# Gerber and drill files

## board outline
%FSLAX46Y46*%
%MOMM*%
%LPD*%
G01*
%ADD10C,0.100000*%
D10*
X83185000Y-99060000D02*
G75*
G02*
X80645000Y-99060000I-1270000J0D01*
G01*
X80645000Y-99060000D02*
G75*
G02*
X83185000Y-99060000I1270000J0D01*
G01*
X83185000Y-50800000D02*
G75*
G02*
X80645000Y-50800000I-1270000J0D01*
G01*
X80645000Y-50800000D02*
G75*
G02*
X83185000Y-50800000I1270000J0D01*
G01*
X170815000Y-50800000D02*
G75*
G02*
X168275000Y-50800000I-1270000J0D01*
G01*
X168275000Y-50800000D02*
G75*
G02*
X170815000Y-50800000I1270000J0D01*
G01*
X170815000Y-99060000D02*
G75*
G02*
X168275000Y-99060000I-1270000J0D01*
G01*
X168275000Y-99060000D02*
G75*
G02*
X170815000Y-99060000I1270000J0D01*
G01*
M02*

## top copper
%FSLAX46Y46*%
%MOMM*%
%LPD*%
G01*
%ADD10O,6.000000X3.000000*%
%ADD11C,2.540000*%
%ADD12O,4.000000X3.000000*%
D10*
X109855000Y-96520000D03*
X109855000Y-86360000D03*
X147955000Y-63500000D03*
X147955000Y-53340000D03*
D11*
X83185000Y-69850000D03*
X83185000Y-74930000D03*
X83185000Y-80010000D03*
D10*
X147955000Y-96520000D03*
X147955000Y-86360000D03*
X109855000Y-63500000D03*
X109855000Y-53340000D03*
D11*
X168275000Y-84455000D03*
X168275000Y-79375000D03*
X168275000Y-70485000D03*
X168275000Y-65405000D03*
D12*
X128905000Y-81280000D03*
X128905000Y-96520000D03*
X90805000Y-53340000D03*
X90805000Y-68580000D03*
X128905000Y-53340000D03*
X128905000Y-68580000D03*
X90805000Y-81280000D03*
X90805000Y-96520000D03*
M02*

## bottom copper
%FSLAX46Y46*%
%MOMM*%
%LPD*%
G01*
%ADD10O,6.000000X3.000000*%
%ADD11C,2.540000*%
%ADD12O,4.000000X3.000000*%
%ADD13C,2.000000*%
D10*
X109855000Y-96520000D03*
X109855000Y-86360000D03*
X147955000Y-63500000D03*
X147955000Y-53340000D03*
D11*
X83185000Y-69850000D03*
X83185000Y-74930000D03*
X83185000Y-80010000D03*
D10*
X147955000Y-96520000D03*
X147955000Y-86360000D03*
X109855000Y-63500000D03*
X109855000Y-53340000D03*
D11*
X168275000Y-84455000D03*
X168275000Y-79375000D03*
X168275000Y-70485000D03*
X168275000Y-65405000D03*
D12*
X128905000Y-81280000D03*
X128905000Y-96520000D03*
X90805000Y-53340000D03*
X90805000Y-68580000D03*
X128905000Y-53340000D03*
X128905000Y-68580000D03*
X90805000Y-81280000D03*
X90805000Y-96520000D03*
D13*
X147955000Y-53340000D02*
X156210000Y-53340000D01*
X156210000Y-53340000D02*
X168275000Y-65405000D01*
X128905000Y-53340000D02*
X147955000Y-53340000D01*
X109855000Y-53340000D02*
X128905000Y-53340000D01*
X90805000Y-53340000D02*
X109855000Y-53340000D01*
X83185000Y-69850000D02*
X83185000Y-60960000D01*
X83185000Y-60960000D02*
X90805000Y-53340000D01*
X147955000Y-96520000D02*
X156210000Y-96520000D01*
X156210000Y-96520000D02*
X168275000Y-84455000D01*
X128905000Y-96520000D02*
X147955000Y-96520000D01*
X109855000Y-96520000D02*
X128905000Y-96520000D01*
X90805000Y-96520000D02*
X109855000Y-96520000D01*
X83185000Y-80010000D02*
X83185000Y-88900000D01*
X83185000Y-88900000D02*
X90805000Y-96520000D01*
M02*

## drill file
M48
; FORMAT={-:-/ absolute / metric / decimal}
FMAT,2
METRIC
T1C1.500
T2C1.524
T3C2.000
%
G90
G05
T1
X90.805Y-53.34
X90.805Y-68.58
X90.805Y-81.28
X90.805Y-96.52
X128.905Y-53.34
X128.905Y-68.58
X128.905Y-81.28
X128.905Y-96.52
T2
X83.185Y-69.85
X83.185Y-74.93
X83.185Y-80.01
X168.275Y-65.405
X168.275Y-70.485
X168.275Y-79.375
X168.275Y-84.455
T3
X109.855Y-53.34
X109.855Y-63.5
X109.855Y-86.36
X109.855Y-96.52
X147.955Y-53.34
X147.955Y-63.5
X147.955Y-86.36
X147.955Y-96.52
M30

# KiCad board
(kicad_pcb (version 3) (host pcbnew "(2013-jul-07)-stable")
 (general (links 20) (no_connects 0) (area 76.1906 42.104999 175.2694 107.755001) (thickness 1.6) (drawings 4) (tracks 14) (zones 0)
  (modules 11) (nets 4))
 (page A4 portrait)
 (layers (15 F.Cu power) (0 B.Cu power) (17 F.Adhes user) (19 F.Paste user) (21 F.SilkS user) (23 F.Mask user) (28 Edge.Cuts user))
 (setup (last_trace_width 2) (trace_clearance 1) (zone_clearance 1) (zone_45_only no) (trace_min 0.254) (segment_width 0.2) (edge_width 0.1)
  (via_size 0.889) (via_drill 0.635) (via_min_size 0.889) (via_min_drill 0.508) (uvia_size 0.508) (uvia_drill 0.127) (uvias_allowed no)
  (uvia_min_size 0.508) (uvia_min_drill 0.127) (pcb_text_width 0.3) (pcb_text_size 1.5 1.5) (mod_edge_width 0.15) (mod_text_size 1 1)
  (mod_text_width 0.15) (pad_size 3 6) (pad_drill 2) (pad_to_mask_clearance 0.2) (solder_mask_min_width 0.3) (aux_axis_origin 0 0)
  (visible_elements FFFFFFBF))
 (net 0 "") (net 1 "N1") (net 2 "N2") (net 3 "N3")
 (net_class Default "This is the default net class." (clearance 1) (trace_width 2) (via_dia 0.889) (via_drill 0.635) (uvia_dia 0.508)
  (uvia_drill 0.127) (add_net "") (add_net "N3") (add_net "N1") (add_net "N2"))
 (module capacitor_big (layer F.Cu) (at 112.395 91.44 270)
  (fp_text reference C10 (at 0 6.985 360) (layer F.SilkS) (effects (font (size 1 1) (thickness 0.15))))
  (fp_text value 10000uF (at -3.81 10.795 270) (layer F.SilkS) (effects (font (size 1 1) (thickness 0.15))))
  (pad 2 thru_hole oval (at 5.08 2.54 270) (size 3 6) (drill 2) (layers *.Cu *.Mask F.SilkS) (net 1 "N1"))
  (pad 1 thru_hole oval (at -5.08 2.54 270) (size 3 6) (drill 2) (layers *.Cu *.Mask F.SilkS) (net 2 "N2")))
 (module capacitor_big (layer F.Cu) (at 150.495 58.42 270)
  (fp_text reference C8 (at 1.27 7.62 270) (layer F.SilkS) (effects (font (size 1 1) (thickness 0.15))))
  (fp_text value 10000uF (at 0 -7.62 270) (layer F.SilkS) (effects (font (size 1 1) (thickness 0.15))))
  (pad 2 thru_hole oval (at 5.08 2.54 270) (size 3 6) (drill 2) (layers *.Cu *.Mask F.SilkS) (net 2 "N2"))
  (pad 1 thru_hole oval (at -5.08 2.54 270) (size 3 6) (drill 2) (layers *.Cu *.Mask F.SilkS) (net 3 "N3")))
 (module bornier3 (layer F.Cu) (at 83.185 74.93 270)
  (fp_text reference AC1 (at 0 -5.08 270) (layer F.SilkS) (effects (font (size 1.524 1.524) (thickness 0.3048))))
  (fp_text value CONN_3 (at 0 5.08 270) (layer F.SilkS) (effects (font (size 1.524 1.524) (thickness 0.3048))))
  (pad 1 thru_hole circle (at -5.08 0 270) (size 2.54 2.54) (drill 1.524) (layers *.Cu *.Mask F.SilkS) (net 3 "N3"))
  (pad 2 thru_hole circle (at 0 0 270) (size 2.54 2.54) (drill 1.524) (layers *.Cu *.Mask F.SilkS) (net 2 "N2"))
  (pad 3 thru_hole circle (at 5.08 0 270) (size 2.54 2.54) (drill 1.524) (layers *.Cu *.Mask F.SilkS) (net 1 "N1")))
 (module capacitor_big (layer F.Cu) (at 150.495 91.44 270)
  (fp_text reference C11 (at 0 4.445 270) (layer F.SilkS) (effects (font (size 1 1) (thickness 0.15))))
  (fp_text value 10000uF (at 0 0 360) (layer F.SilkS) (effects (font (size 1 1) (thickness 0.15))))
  (pad 2 thru_hole oval (at 5.08 2.54 270) (size 3 6) (drill 2) (layers *.Cu *.Mask F.SilkS) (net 1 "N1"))
  (pad 1 thru_hole oval (at -5.08 2.54 270) (size 3 6) (drill 2) (layers *.Cu *.Mask F.SilkS) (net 2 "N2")))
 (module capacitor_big (layer F.Cu) (at 112.395 58.42 270)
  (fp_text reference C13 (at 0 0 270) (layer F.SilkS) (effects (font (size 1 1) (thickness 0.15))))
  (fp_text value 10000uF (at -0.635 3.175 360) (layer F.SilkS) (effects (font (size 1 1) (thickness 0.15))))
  (pad 2 thru_hole oval (at 5.08 2.54 270) (size 3 6) (drill 2) (layers *.Cu *.Mask F.SilkS) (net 2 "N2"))
  (pad 1 thru_hole oval (at -5.08 2.54 270) (size 3 6) (drill 2) (layers *.Cu *.Mask F.SilkS) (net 3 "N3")))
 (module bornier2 (layer F.Cu) (at 168.275 81.915 90)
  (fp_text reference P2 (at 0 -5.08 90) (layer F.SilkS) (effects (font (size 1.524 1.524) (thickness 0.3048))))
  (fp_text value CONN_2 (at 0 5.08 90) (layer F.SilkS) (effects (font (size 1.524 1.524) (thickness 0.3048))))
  (pad 1 thru_hole circle (at -2.54 0 90) (size 2.54 2.54) (drill 1.524) (layers *.Cu *.Mask F.SilkS) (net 1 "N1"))
  (pad 2 thru_hole circle (at 2.54 0 90) (size 2.54 2.54) (drill 1.524) (layers *.Cu *.Mask F.SilkS) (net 2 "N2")))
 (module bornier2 (layer F.Cu) (at 168.275 67.945 90)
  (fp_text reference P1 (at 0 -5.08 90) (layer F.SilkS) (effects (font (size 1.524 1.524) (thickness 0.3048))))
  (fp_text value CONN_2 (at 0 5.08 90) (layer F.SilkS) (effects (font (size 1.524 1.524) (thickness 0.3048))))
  (pad 1 thru_hole circle (at -2.54 0 90) (size 2.54 2.54) (drill 1.524) (layers *.Cu *.Mask F.SilkS) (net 2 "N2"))
  (pad 2 thru_hole circle (at 2.54 0 90) (size 2.54 2.54) (drill 1.524) (layers *.Cu *.Mask F.SilkS) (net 3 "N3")))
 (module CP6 (layer F.Cu) (at 128.905 88.9 270)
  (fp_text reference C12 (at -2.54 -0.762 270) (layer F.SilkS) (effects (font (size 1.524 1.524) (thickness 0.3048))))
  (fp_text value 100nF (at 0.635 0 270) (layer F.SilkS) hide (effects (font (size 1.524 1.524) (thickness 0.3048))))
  (pad 1 thru_hole oval (at -7.62 0 270) (size 3 4) (drill 1.5) (layers *.Cu *.Mask F.SilkS) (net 2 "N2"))
  (pad 2 thru_hole oval (at 7.62 0 270) (size 3 4) (drill 1.5) (layers *.Cu *.Mask F.SilkS) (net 1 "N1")))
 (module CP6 (layer F.Cu) (at 90.805 60.96 270)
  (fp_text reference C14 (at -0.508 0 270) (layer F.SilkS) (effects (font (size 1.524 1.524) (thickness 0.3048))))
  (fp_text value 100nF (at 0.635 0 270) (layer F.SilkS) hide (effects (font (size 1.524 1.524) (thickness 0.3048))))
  (pad 1 thru_hole oval (at -7.62 0 270) (size 3 4) (drill 1.5) (layers *.Cu *.Mask F.SilkS) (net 3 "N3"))
  (pad 2 thru_hole oval (at 7.62 0 270) (size 3 4) (drill 1.5) (layers *.Cu *.Mask F.SilkS) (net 2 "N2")))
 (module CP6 (layer F.Cu) (at 128.905 60.96 270)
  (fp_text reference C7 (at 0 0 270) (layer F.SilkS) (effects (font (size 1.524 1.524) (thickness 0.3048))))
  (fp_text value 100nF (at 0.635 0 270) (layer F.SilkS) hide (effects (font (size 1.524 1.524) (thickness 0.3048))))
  (pad 1 thru_hole oval (at -7.62 0 270) (size 3 4) (drill 1.5) (layers *.Cu *.Mask F.SilkS) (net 3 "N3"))
  (pad 2 thru_hole oval (at 7.62 0 270) (size 3 4) (drill 1.5) (layers *.Cu *.Mask F.SilkS) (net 2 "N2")))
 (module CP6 (layer F.Cu) (at 90.805 88.9 270)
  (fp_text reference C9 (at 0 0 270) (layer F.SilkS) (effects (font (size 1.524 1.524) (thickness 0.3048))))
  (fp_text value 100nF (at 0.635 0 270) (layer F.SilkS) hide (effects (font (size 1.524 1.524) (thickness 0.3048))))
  (pad 1 thru_hole oval (at -7.62 0 270) (size 3 4) (drill 1.5) (layers *.Cu *.Mask F.SilkS) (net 2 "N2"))
  (pad 2 thru_hole oval (at 7.62 0 270) (size 3 4) (drill 1.5) (layers *.Cu *.Mask F.SilkS) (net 1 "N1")))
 (gr_circle (center 81.915 99.06) (end 83.185 99.06) (layer Edge.Cuts) (width 0.1))
 (gr_circle (center 81.915 50.8) (end 83.185 50.8) (layer Edge.Cuts) (width 0.1))
 (gr_circle (center 169.545 50.8) (end 170.815 50.8) (layer Edge.Cuts) (width 0.1))
 (gr_circle (center 169.545 99.06) (end 170.815 99.06) (layer Edge.Cuts) (width 0.1))
 (segment (start 147.955 53.34) (end 156.21 53.34) (width 2) (layer B.Cu) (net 3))
 (segment (start 156.21 53.34) (end 168.275 65.405) (width 2) (layer B.Cu) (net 3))
 (segment (start 128.905 53.34) (end 147.955 53.34) (width 2) (layer B.Cu) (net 3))
 (segment (start 109.855 53.34) (end 128.905 53.34) (width 2) (layer B.Cu) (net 3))
 (segment (start 90.805 53.34) (end 109.855 53.34) (width 2) (layer B.Cu) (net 3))
 (segment (start 83.185 69.85) (end 83.185 60.96) (width 2) (layer B.Cu) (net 3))
 (segment (start 83.185 60.96) (end 90.805 53.34) (width 2) (layer B.Cu) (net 3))
 (segment (start 147.955 96.52) (end 156.21 96.52) (width 2) (layer B.Cu) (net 1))
 (segment (start 156.21 96.52) (end 168.275 84.455) (width 2) (layer B.Cu) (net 1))
 (segment (start 128.905 96.52) (end 147.955 96.52) (width 2) (layer B.Cu) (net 1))
 (segment (start 109.855 96.52) (end 128.905 96.52) (width 2) (layer B.Cu) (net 1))
 (segment (start 90.805 96.52) (end 109.855 96.52) (width 2) (layer B.Cu) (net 1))
 (segment (start 83.185 80.01) (end 83.185 88.9) (width 2) (layer B.Cu) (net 1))
 (segment (start 83.185 88.9) (end 90.805 96.52) (width 2) (layer B.Cu) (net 1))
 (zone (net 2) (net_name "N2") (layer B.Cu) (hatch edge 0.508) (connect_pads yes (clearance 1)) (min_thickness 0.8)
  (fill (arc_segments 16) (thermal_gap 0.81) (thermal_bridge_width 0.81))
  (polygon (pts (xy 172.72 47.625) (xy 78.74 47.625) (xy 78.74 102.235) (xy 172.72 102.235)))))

